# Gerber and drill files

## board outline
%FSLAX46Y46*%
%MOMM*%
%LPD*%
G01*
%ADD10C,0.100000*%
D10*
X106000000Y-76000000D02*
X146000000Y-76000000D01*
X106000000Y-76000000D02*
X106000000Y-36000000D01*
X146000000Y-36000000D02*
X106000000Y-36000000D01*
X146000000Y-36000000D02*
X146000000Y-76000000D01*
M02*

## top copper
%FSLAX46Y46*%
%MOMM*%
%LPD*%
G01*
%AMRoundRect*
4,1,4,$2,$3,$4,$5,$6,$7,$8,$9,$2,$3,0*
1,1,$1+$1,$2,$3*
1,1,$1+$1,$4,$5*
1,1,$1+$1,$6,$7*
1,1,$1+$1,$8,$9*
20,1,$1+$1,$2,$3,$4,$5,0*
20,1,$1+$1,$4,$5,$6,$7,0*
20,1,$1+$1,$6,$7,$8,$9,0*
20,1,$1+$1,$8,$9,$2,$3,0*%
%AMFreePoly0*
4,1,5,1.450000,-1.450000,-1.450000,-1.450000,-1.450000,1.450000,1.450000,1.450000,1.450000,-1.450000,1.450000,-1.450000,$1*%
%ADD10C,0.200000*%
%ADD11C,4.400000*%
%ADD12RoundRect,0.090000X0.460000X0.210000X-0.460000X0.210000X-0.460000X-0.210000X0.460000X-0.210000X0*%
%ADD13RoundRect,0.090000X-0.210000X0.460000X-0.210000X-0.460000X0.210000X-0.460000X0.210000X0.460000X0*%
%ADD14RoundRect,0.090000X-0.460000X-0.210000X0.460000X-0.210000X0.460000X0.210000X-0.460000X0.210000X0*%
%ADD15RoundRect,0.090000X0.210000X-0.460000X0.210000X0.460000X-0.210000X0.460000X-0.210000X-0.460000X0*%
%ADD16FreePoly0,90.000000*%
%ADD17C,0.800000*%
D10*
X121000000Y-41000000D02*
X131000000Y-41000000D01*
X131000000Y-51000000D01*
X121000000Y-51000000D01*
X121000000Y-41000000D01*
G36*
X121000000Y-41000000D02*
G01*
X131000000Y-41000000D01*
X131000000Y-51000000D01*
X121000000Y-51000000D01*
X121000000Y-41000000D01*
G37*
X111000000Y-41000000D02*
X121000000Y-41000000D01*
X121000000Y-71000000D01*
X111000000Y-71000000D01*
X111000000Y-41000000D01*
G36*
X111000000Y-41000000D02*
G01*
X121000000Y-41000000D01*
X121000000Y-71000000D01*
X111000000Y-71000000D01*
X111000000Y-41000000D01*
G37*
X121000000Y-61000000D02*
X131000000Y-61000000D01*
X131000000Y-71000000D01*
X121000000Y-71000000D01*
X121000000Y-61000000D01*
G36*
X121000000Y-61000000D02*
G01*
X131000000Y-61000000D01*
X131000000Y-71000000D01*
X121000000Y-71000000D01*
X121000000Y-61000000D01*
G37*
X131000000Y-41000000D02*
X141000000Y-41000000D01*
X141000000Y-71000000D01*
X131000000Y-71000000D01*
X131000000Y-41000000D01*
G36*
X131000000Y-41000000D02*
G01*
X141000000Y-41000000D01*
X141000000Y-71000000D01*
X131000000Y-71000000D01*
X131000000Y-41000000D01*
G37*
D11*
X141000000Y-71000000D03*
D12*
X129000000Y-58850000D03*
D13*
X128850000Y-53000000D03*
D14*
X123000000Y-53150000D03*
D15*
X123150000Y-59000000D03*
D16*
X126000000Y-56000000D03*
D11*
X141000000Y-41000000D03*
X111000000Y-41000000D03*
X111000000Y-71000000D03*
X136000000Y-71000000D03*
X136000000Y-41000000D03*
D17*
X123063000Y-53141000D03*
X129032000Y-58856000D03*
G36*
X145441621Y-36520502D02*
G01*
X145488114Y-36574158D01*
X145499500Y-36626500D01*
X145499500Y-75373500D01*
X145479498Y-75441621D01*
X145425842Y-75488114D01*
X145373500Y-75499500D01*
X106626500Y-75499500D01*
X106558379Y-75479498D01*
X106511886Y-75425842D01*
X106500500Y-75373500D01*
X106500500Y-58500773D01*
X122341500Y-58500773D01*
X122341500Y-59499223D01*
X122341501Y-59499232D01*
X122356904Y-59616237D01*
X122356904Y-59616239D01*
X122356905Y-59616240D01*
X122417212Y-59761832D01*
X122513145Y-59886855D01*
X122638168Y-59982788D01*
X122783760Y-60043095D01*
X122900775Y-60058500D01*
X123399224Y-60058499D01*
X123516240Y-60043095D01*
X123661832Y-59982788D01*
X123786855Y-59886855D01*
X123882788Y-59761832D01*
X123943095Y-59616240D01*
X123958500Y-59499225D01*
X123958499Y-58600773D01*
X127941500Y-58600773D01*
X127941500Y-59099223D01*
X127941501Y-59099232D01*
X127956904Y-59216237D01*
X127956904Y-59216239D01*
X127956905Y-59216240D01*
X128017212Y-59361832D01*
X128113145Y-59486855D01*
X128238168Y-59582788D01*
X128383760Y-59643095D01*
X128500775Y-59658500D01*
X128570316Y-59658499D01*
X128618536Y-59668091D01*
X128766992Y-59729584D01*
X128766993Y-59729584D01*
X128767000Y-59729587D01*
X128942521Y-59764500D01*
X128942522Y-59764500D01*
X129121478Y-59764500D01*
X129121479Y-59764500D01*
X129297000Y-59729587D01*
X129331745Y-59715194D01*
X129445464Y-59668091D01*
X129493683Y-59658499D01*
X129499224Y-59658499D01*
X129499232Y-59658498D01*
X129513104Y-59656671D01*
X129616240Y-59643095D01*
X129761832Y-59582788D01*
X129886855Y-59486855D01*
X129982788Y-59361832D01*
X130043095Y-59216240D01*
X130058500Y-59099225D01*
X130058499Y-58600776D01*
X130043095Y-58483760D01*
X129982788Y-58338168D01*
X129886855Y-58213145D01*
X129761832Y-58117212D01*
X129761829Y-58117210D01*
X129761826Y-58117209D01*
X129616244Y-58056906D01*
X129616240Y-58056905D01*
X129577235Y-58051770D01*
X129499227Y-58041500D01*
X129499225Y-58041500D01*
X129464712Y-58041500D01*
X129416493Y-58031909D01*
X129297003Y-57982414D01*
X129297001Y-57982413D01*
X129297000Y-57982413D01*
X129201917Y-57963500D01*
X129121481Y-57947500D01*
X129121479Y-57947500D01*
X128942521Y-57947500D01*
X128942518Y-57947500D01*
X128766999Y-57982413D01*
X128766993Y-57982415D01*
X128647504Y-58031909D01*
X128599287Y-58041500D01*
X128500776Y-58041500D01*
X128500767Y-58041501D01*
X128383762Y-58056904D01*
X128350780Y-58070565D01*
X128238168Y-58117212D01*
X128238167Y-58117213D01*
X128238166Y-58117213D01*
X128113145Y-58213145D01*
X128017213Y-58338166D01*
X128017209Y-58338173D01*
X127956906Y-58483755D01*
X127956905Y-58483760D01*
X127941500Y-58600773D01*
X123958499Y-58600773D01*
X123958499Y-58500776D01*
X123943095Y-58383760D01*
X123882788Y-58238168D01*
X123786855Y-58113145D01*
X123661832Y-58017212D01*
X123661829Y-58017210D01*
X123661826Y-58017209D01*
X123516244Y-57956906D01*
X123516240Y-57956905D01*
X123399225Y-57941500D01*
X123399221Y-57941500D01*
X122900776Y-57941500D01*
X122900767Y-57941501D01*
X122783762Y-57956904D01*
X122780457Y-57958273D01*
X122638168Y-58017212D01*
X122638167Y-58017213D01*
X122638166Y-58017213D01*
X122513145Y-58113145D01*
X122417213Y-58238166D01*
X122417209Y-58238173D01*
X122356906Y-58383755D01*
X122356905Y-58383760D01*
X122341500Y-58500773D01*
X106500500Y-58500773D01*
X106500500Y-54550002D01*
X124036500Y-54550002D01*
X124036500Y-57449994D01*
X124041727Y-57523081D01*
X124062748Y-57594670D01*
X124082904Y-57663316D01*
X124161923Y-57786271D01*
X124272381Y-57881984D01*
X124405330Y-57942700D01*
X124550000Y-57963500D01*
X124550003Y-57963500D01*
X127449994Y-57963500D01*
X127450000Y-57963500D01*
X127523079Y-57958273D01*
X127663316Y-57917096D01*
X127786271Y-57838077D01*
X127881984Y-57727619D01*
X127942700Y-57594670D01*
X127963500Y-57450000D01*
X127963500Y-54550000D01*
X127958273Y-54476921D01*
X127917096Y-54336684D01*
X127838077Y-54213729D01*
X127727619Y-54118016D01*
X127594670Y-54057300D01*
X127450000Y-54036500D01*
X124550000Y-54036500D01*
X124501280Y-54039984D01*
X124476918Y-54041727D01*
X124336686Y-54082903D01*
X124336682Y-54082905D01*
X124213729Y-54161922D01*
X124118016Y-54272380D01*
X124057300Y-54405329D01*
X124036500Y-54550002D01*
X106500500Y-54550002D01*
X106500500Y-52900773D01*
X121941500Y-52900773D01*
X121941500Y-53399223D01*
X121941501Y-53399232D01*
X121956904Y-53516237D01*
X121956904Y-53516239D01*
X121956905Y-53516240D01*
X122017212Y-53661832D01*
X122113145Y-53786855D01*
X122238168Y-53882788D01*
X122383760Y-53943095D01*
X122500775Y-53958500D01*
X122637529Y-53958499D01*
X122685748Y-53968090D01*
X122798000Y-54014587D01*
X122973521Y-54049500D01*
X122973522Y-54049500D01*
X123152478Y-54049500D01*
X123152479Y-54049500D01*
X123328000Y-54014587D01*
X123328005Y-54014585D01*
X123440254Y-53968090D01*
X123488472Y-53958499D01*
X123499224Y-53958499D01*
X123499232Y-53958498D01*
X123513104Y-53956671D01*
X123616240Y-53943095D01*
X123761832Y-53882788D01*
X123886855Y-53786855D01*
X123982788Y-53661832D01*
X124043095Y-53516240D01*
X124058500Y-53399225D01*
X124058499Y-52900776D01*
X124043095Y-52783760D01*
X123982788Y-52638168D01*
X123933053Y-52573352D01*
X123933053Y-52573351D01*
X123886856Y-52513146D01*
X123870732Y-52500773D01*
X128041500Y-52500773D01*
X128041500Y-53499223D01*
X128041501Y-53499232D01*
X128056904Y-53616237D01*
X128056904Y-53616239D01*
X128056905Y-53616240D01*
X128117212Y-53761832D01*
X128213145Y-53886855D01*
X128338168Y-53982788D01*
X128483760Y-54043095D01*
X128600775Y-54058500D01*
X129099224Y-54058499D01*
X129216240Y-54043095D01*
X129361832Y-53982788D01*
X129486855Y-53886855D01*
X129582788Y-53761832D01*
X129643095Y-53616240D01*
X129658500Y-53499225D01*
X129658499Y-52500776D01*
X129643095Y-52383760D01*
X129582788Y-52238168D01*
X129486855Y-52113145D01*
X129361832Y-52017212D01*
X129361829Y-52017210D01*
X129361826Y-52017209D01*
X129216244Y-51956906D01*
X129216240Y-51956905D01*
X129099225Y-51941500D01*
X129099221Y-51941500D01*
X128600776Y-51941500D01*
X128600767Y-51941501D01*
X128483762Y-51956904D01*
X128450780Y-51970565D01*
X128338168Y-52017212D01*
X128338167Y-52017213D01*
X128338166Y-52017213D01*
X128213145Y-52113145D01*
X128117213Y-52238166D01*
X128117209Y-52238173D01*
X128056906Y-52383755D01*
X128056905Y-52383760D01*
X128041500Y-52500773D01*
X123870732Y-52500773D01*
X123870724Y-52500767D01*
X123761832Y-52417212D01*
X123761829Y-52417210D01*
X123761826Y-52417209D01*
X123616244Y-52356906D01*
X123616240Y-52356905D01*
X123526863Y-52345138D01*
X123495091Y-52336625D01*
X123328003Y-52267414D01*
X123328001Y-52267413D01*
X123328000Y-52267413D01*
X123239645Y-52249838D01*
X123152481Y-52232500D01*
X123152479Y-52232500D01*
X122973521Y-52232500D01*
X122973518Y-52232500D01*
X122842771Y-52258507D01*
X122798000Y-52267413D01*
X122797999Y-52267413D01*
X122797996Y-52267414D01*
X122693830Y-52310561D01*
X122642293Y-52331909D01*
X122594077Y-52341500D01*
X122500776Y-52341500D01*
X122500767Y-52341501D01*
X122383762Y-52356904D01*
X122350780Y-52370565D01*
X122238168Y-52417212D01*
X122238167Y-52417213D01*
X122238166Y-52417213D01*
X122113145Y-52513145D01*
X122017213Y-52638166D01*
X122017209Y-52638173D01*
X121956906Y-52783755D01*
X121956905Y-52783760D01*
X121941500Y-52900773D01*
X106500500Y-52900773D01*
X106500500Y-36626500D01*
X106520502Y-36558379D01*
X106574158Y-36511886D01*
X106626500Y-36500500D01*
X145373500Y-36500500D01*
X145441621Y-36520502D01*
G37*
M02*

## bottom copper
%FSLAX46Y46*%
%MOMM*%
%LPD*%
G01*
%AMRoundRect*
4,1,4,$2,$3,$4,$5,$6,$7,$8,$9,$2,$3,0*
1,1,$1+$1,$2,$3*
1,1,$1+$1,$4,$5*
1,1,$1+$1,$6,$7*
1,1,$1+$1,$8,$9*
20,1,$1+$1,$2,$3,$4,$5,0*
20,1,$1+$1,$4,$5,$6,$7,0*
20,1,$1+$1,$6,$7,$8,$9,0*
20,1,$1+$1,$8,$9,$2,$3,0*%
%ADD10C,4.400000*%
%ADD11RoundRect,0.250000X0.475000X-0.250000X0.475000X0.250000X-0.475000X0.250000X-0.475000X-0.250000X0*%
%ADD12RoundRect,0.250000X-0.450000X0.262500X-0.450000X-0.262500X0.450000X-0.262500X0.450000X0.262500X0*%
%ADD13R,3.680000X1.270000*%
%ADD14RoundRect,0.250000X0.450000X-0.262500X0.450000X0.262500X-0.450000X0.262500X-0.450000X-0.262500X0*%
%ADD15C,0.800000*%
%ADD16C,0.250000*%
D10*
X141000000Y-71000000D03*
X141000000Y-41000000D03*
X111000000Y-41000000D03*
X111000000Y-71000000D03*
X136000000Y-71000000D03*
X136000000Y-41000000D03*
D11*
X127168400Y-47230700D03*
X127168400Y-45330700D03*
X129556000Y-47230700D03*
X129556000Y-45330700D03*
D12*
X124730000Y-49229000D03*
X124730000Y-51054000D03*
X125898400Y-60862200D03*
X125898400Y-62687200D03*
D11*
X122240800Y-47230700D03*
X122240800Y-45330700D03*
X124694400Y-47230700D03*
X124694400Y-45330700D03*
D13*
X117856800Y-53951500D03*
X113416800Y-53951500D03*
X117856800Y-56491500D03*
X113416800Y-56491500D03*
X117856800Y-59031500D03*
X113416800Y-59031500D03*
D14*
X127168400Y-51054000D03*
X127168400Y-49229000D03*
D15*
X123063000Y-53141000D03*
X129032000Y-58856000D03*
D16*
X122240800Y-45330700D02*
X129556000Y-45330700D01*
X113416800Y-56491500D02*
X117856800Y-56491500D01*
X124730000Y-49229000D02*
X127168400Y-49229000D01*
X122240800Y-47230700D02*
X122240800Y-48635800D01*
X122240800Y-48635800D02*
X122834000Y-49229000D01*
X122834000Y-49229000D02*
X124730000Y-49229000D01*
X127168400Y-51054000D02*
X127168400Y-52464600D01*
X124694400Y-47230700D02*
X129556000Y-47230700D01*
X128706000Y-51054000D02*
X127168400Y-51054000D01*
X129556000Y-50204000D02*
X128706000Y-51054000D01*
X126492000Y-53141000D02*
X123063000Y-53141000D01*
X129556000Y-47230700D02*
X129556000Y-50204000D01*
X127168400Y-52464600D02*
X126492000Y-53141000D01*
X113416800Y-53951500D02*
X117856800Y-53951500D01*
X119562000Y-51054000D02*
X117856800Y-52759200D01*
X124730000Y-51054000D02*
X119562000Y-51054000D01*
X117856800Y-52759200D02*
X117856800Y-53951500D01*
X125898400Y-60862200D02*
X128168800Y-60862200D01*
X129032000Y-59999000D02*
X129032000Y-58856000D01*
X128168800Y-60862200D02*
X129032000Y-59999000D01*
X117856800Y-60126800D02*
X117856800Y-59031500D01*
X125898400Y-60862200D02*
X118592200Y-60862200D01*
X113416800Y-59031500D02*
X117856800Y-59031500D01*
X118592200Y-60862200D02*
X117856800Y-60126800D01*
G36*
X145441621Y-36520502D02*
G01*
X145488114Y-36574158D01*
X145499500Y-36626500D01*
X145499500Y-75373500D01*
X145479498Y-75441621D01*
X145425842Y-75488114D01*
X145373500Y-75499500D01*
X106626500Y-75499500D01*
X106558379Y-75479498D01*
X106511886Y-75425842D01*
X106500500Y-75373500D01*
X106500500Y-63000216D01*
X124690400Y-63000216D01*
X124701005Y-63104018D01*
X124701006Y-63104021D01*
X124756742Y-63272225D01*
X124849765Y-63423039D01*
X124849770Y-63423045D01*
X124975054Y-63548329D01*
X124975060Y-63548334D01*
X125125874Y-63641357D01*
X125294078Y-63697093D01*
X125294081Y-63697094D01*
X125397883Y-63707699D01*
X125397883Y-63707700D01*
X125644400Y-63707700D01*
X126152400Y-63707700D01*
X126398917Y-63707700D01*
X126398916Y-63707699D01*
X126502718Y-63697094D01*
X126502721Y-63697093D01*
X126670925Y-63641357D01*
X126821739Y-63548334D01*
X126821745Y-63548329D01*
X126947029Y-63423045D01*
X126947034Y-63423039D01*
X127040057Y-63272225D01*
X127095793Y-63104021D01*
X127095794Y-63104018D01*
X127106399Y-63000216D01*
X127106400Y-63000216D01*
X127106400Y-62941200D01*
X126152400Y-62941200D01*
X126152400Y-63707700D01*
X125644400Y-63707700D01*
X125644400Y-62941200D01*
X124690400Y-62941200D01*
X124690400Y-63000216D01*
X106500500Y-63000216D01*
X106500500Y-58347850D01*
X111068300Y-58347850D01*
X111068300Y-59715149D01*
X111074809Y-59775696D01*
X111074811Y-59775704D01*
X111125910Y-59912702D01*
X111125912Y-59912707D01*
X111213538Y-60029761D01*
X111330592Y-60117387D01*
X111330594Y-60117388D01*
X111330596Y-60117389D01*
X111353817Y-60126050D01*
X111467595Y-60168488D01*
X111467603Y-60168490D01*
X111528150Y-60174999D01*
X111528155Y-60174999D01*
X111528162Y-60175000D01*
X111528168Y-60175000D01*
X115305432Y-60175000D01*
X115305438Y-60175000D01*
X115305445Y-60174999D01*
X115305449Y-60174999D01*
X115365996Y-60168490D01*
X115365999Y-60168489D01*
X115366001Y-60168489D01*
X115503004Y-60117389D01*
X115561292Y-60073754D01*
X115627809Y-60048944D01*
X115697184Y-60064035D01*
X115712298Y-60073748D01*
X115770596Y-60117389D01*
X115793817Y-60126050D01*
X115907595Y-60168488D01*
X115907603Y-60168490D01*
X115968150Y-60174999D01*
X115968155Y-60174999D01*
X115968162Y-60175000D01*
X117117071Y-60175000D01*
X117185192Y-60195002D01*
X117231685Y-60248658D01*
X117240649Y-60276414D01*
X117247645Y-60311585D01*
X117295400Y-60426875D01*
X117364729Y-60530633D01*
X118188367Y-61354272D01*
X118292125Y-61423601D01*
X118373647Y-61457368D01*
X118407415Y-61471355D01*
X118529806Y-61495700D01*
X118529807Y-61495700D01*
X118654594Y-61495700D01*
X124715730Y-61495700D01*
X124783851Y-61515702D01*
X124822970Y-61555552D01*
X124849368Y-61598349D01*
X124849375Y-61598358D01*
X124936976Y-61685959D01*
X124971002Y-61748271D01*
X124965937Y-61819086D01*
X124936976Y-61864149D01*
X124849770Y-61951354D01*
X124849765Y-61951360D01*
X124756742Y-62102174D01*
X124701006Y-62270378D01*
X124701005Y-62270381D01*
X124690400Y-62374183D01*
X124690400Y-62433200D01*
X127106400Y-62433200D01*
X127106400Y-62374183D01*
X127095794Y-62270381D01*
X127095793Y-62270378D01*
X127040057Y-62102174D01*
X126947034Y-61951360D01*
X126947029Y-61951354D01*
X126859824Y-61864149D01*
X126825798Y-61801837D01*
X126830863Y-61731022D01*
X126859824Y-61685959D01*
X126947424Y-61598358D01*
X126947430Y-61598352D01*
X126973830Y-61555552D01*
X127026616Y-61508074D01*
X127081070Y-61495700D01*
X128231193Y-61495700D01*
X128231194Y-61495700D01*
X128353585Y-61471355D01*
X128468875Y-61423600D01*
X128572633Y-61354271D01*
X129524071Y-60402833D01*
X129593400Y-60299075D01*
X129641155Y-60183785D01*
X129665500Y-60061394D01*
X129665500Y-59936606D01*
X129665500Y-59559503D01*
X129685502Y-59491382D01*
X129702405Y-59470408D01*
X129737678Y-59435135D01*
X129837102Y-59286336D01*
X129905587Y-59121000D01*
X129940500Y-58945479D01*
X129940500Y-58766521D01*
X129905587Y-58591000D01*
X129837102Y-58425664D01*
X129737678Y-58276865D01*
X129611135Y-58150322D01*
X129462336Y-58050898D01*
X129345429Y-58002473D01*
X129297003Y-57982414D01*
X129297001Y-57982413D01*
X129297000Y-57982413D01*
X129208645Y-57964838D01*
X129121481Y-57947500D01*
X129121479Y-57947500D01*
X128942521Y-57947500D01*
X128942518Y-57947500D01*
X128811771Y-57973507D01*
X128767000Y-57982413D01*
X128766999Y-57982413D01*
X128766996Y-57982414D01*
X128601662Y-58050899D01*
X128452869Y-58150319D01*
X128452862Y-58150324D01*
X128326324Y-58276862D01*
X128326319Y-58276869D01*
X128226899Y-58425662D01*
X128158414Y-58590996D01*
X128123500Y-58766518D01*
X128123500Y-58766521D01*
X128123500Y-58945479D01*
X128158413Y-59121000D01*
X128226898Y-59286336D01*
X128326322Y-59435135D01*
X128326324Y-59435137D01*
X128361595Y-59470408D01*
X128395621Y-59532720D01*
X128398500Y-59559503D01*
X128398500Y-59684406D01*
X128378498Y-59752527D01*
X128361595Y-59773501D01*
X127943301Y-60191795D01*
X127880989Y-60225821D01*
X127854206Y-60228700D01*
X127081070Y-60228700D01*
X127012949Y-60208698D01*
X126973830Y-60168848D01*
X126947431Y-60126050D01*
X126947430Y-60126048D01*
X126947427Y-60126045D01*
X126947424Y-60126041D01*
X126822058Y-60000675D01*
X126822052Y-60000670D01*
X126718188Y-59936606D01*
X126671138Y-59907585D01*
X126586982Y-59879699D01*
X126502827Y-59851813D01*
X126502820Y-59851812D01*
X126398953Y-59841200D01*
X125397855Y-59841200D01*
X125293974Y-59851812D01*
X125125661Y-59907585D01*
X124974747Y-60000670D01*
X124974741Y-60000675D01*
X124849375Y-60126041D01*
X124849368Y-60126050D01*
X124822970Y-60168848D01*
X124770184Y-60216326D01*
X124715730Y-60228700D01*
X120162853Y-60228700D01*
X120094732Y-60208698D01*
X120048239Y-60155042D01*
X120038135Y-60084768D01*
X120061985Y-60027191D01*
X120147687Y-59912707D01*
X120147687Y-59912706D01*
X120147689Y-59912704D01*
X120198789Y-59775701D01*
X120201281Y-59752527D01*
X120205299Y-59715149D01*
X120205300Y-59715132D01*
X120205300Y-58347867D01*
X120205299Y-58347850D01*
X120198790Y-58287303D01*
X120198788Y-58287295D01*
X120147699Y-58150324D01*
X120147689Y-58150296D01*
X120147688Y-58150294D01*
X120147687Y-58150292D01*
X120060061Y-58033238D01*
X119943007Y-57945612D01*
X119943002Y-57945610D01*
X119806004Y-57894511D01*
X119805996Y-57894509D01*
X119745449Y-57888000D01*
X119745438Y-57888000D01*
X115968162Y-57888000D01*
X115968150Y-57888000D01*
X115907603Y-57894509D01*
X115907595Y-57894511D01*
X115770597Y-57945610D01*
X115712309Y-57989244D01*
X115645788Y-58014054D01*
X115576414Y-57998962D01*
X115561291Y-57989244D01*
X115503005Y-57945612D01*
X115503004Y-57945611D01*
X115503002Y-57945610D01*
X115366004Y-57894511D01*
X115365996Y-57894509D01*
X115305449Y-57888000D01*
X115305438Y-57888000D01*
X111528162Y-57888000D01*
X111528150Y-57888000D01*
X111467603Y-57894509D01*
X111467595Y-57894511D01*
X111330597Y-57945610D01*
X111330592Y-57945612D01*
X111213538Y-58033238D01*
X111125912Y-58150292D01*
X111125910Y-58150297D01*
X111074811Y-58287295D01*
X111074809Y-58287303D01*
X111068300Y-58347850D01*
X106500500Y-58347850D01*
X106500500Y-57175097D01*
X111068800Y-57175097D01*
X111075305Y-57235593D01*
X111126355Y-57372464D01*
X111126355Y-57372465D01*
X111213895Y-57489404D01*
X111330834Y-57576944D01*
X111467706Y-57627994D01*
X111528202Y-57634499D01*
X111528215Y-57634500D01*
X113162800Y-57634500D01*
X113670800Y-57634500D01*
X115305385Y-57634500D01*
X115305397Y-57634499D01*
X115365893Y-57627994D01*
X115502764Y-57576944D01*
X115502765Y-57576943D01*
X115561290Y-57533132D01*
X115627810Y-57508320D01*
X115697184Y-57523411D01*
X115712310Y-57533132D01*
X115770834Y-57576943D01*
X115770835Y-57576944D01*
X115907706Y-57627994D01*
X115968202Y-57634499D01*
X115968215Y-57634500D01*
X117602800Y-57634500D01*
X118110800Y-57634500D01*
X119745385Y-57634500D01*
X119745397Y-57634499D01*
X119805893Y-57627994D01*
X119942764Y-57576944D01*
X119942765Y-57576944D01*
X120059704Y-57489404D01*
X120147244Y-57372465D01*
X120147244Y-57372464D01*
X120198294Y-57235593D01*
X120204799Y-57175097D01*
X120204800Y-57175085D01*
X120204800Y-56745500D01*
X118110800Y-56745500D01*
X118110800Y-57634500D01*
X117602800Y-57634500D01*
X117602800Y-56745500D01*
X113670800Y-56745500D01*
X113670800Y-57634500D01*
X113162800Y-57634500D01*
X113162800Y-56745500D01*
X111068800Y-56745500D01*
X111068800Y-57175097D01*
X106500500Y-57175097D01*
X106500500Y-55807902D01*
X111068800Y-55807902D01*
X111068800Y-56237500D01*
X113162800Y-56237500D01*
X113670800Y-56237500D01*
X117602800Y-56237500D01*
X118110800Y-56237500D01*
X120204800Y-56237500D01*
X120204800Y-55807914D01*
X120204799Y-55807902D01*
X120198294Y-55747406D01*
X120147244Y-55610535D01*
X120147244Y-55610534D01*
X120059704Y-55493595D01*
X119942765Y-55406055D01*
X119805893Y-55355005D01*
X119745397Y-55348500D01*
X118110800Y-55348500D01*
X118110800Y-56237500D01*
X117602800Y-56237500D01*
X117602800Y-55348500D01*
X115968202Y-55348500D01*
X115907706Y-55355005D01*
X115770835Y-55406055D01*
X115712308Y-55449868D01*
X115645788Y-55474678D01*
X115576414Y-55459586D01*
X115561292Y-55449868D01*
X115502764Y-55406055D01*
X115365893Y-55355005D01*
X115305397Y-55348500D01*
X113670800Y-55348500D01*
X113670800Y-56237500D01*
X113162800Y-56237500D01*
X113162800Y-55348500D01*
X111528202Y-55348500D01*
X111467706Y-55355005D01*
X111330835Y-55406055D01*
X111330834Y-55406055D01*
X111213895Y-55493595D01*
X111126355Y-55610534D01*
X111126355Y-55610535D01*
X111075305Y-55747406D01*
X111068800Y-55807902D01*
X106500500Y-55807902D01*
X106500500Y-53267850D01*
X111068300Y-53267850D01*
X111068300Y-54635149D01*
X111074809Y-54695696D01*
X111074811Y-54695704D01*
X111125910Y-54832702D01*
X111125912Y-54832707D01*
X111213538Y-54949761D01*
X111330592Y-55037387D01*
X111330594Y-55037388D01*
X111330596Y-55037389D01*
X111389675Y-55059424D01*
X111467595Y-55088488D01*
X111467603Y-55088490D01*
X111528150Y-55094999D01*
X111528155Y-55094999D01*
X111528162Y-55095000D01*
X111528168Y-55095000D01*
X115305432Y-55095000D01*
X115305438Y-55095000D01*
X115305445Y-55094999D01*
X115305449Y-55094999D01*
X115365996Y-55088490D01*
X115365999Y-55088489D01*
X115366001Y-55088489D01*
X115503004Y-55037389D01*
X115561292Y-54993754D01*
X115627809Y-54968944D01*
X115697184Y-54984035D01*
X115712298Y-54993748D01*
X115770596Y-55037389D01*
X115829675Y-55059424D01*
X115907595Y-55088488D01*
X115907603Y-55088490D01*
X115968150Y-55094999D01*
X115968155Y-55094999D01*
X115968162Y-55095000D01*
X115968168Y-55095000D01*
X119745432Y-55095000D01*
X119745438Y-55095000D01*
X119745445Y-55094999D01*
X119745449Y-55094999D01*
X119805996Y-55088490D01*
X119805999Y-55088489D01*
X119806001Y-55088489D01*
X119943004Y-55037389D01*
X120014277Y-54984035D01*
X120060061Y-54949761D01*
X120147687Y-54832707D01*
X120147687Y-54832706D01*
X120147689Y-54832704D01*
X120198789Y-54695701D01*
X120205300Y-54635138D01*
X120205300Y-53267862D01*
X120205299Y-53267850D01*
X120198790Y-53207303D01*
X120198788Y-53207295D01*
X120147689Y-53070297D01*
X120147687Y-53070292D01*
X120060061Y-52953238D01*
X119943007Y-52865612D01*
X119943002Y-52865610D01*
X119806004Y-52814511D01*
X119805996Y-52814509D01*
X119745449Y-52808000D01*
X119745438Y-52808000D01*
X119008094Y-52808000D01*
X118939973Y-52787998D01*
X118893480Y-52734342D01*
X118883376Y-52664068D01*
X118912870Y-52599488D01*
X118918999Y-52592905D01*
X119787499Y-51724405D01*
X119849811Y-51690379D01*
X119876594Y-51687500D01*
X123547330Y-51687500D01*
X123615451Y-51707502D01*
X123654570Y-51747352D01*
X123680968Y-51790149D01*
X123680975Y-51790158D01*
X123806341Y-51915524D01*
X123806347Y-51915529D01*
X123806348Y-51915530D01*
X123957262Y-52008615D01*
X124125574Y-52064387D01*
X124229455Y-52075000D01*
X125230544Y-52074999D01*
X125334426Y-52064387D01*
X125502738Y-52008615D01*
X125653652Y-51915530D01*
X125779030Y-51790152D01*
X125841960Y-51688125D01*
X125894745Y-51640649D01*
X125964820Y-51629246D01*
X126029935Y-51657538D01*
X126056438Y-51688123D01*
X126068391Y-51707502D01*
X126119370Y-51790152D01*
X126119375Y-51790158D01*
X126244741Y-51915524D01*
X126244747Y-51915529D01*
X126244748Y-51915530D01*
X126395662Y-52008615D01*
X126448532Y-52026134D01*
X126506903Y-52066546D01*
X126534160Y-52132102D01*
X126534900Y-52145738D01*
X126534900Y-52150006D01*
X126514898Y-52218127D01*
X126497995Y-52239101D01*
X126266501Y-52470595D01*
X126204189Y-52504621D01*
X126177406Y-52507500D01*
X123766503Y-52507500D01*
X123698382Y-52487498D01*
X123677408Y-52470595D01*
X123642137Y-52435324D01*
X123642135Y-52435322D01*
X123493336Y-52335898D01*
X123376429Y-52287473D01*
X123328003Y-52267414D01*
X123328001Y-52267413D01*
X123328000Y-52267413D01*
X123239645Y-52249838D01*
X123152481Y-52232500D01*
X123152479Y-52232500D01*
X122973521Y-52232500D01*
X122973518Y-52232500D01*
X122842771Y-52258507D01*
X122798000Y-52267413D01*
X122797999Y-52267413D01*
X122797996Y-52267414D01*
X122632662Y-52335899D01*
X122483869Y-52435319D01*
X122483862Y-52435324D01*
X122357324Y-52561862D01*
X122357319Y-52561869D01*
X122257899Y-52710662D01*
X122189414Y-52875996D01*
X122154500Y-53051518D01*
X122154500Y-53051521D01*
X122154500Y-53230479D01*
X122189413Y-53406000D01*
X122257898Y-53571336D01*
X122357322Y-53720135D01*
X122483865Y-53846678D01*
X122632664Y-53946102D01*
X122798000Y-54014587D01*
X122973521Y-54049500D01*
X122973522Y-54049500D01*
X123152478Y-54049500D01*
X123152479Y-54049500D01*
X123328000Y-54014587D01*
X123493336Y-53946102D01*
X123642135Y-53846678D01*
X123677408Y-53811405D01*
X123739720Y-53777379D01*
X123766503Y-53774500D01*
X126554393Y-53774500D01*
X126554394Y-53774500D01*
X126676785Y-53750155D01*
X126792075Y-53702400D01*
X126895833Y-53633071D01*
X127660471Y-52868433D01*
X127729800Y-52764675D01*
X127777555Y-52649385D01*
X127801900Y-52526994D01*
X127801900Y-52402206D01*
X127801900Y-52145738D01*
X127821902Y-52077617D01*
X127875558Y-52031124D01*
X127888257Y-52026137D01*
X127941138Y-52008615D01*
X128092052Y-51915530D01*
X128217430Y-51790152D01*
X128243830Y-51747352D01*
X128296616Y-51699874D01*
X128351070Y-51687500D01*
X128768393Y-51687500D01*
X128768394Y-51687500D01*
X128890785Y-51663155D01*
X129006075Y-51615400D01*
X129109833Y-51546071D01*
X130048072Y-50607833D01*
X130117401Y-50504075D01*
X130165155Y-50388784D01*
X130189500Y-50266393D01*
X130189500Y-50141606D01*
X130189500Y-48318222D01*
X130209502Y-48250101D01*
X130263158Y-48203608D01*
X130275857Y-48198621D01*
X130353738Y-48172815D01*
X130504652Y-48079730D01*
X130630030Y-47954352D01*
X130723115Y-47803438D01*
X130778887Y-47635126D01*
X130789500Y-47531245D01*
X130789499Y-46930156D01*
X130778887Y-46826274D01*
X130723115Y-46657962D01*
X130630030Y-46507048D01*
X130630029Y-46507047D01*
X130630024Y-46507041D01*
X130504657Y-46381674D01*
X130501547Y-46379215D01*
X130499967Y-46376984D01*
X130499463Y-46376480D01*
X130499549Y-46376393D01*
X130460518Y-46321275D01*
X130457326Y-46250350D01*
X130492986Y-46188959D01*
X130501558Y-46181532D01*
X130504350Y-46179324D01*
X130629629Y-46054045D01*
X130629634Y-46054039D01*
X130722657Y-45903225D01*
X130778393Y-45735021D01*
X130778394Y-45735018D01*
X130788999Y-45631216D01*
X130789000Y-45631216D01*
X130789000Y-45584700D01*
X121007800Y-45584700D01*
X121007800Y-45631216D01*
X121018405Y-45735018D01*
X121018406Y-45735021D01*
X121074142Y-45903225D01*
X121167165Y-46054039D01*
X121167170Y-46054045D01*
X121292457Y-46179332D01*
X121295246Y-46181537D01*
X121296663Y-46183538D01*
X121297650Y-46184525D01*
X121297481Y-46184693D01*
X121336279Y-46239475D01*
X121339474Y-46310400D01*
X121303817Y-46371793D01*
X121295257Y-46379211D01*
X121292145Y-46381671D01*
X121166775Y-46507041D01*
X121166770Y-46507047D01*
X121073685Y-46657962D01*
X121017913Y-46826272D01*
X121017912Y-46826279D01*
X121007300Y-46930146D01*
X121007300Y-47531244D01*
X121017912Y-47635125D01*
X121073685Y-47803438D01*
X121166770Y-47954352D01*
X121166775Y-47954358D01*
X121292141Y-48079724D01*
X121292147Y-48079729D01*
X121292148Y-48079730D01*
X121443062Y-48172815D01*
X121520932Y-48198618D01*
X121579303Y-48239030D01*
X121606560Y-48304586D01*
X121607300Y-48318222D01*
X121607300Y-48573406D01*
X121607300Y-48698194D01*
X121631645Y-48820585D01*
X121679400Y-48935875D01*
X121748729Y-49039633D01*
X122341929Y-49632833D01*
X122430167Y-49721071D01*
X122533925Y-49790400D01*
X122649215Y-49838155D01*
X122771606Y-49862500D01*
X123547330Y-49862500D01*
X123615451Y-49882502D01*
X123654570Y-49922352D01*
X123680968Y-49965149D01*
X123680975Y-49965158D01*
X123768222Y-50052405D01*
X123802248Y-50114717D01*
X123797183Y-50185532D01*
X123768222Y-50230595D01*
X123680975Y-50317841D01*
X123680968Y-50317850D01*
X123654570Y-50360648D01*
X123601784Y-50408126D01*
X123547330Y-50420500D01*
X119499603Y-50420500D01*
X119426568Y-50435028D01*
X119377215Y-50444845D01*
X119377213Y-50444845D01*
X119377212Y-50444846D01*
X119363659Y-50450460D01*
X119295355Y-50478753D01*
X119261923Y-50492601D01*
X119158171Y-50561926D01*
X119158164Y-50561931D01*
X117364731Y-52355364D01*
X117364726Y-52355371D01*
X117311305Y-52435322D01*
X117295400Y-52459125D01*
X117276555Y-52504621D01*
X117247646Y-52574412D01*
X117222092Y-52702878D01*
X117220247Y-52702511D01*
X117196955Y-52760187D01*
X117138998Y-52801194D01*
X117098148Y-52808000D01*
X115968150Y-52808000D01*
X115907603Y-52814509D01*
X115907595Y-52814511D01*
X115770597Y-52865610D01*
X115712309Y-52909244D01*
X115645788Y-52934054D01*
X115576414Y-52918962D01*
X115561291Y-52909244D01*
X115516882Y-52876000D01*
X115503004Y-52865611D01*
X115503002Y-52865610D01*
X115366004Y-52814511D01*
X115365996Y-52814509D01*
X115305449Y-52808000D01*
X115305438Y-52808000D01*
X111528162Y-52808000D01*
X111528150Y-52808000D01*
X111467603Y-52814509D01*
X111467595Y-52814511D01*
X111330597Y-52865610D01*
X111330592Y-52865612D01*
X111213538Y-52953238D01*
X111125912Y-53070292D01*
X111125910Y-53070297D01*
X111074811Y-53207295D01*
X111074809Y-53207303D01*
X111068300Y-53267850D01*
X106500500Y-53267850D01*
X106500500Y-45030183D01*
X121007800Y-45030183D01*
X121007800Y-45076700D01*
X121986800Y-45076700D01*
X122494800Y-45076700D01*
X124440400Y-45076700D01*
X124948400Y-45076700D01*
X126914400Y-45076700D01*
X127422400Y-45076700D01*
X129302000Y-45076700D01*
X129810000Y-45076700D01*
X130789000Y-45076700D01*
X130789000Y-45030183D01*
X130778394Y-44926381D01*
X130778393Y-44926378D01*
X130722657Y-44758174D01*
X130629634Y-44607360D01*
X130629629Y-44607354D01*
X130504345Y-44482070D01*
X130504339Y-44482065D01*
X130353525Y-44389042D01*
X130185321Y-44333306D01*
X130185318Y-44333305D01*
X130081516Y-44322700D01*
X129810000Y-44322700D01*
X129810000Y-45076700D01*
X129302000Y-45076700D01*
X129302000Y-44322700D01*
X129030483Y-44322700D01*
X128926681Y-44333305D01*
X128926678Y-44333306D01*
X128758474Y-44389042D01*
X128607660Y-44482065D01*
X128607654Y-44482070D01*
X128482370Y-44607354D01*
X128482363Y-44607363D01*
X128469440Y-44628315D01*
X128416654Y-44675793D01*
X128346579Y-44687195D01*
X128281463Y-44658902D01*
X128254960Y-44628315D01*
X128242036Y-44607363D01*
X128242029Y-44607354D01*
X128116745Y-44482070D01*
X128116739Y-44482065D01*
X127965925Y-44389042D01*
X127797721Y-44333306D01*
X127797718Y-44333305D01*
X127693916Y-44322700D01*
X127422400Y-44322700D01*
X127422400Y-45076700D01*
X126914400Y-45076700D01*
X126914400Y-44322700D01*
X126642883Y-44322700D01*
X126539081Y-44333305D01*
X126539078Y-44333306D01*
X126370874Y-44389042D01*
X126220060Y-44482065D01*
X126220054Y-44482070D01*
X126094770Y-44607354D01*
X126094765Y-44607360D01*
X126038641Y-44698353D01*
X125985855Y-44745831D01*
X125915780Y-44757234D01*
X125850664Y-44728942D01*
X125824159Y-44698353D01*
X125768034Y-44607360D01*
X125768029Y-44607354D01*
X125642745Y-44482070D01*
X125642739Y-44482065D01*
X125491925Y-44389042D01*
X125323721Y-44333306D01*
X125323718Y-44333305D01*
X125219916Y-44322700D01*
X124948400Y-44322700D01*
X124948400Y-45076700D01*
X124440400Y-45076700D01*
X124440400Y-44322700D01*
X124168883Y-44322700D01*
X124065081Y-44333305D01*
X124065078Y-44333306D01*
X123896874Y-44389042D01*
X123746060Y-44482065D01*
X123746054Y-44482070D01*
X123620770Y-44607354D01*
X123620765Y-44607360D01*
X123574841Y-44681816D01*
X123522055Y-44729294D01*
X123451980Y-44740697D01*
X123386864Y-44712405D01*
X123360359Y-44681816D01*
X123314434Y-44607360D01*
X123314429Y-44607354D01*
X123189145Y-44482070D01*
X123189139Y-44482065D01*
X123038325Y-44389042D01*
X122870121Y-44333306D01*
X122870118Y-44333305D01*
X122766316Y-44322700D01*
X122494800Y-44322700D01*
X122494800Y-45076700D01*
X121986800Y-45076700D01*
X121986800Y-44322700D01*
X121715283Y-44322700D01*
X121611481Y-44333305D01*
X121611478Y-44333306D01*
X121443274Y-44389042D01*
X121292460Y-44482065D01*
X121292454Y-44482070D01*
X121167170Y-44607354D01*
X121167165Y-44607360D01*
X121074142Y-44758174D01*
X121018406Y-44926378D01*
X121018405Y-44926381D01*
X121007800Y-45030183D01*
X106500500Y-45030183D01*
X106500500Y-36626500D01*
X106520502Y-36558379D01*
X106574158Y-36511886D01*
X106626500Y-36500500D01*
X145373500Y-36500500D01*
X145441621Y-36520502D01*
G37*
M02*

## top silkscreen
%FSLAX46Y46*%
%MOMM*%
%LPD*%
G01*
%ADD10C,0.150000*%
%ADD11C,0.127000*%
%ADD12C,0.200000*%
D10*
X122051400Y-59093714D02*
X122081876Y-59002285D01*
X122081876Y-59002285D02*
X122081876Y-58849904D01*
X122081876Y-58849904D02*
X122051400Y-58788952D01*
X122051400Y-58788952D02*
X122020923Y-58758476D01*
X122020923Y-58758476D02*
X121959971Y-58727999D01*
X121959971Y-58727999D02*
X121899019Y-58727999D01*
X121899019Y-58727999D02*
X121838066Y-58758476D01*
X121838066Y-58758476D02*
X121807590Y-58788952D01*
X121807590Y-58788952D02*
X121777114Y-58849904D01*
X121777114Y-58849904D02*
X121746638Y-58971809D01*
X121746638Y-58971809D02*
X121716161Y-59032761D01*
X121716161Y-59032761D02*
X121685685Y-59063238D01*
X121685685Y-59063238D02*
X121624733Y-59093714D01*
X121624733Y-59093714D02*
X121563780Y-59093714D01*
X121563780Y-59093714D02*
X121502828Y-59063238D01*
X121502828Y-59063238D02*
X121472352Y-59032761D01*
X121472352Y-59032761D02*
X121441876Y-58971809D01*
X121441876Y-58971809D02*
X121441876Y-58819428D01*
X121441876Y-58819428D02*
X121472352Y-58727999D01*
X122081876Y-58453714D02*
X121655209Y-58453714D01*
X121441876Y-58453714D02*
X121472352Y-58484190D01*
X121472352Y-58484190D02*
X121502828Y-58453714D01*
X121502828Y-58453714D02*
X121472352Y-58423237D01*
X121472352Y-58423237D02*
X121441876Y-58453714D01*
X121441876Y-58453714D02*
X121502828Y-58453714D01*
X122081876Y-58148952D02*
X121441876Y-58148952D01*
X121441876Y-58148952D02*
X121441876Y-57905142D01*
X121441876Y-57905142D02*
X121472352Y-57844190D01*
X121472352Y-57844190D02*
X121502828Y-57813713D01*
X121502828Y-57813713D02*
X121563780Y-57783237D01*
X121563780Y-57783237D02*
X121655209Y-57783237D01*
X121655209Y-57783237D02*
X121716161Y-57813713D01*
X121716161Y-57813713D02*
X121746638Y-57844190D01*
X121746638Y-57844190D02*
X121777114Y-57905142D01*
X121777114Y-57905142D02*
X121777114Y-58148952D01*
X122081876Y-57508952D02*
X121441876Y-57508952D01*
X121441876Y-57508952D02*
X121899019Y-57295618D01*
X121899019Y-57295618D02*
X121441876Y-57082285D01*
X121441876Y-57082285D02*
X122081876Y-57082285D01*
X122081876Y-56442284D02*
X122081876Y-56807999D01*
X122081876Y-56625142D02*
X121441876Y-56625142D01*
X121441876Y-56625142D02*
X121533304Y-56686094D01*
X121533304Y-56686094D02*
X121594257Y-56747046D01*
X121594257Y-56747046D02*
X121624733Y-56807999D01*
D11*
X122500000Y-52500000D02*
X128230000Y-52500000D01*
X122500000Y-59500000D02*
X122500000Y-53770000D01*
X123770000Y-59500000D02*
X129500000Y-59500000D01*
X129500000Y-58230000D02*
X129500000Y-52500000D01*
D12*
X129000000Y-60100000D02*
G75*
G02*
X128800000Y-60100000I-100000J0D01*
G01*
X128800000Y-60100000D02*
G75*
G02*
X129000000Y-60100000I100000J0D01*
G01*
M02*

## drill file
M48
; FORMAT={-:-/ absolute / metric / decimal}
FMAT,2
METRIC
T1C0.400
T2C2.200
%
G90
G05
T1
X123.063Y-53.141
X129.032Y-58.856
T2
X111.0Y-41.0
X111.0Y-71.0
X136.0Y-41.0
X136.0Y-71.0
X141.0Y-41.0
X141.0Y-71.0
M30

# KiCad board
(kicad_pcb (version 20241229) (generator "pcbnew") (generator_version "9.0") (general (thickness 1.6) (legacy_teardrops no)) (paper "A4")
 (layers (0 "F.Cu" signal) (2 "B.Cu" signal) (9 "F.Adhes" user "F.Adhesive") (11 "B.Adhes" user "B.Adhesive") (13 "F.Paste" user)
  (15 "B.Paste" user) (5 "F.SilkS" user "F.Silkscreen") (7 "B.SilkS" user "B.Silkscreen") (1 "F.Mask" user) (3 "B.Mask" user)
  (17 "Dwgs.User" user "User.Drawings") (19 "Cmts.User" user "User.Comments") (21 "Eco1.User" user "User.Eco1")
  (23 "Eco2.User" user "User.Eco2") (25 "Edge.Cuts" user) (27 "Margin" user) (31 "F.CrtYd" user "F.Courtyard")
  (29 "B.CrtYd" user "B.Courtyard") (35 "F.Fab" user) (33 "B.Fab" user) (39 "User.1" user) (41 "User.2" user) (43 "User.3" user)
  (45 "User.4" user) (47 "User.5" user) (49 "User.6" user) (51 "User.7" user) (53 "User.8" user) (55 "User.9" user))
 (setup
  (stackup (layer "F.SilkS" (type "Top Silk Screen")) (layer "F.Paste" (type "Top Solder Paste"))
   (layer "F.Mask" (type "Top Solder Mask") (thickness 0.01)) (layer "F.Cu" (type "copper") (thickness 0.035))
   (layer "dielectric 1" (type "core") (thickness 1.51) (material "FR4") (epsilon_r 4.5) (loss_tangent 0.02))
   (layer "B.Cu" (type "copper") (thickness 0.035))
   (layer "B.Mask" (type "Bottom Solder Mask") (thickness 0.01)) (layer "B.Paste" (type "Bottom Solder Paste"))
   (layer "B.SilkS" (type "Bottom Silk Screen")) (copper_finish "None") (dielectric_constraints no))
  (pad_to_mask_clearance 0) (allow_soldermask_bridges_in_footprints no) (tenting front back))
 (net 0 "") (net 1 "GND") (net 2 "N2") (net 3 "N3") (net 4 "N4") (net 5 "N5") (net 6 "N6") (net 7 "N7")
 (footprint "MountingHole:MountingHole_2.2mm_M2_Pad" (layer "F.Cu") (at 141 71)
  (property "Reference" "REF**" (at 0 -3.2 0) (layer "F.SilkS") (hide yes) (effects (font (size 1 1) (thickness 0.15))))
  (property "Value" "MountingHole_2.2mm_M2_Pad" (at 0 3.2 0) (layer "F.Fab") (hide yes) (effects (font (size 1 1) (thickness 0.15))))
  (pad "1" thru_hole circle (at 0 0) (size 4.4 4.4) (drill 2.2) (layers "*.Cu" "*.Mask") (remove_unused_layers no) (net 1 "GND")
   (zone_connect 2)))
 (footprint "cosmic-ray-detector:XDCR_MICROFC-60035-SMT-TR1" (layer "F.Cu") (at 126 56 90)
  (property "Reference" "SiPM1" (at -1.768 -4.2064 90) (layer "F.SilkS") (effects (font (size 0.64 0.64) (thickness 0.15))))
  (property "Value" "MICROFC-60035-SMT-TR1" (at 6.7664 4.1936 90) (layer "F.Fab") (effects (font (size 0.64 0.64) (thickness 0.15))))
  (fp_line (start 3.5 -3.5) (end 3.5 2.23) (stroke (width 0.127) (type solid)) (layer "F.SilkS"))
  (fp_line (start -3.5 -3.5) (end 2.23 -3.5) (stroke (width 0.127) (type solid)) (layer "F.SilkS"))
  (fp_line (start -3.5 -2.23) (end -3.5 3.5) (stroke (width 0.127) (type solid)) (layer "F.SilkS"))
  (fp_line (start -2.23 3.5) (end 3.5 3.5) (stroke (width 0.127) (type solid)) (layer "F.SilkS"))
  (fp_circle (center -4.1 2.9) (end -4 2.9) (stroke (width 0.2) (type solid)) (fill no) (layer "F.SilkS"))
  (pad "1" smd roundrect (at -2.85 3 180) (size 1.1 0.6) (layers "F.Cu" "F.Mask" "F.Paste") (roundrect_rratio 0.15) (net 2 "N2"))
  (pad "2" smd roundrect (at 3 2.85 270) (size 1.1 0.6) (layers "F.Cu" "F.Mask" "F.Paste") (roundrect_rratio 0.15) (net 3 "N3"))
  (pad "3" smd roundrect (at 2.85 -3) (size 1.1 0.6) (layers "F.Cu" "F.Mask" "F.Paste") (roundrect_rratio 0.15) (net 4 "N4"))
  (pad "4" smd roundrect (at -3 -2.85 90) (size 1.1 0.6) (layers "F.Cu" "F.Mask" "F.Paste") (roundrect_rratio 0.15))
  (pad "5" smd custom (at 0 0 90) (size 2.9 2.9) (layers "F.Cu") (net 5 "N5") (zone_connect 0) (options (clearance outline) (anchor rect))
   (primitives)))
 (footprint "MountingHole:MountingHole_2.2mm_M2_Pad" (layer "F.Cu") (at 141 41)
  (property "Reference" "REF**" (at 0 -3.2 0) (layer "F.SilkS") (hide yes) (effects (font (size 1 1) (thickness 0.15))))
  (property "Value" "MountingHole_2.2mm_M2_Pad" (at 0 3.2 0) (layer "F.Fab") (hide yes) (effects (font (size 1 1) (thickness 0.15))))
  (pad "1" thru_hole circle (at 0 0) (size 4.4 4.4) (drill 2.2) (layers "*.Cu" "*.Mask") (remove_unused_layers no) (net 1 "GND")
   (zone_connect 2)))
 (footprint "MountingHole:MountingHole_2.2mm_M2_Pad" (layer "F.Cu") (at 111 41)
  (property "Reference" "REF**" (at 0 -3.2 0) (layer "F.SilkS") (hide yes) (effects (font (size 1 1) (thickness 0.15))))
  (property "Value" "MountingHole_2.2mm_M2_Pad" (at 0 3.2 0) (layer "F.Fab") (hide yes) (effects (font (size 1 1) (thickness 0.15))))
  (pad "1" thru_hole circle (at 0 0) (size 4.4 4.4) (drill 2.2) (layers "*.Cu" "*.Mask") (remove_unused_layers no) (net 1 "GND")
   (zone_connect 2)))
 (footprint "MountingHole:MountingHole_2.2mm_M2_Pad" (layer "F.Cu") (at 111 71)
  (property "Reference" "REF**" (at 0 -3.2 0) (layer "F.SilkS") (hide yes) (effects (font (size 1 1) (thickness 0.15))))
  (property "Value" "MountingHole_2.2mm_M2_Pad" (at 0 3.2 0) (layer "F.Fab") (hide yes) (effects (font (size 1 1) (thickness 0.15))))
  (pad "1" thru_hole circle (at 0 0) (size 4.4 4.4) (drill 2.2) (layers "*.Cu" "*.Mask") (remove_unused_layers no) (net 1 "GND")
   (zone_connect 2)))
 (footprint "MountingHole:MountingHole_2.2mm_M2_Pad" (layer "F.Cu") (at 136 71)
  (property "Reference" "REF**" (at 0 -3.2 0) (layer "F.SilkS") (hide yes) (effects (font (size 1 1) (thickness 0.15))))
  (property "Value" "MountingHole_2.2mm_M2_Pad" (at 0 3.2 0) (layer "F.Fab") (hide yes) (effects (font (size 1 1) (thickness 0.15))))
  (pad "1" thru_hole circle (at 0 0) (size 4.4 4.4) (drill 2.2) (layers "*.Cu" "*.Mask") (remove_unused_layers no) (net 1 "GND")
   (zone_connect 2)))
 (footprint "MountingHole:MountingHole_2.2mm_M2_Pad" (layer "F.Cu") (at 136 41)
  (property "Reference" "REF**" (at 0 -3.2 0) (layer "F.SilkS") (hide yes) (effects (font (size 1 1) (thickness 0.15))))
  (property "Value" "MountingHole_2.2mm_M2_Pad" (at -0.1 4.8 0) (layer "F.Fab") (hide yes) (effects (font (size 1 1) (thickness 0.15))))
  (pad "1" thru_hole circle (at 0 0) (size 4.4 4.4) (drill 2.2) (layers "*.Cu" "*.Mask") (remove_unused_layers no) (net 1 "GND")
   (zone_connect 2)))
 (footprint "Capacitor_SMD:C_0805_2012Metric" (layer "B.Cu") (at 127.1684 46.2807 90)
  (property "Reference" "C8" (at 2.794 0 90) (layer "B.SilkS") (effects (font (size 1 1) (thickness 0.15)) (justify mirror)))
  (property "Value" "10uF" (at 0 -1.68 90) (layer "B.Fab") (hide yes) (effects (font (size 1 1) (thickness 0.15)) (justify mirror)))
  (pad "1" smd roundrect (at -0.95 0 90) (size 1 1.45) (layers "B.Cu" "B.Mask" "B.Paste") (roundrect_rratio 0.25) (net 4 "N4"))
  (pad "2" smd roundrect (at 0.95 0 90) (size 1 1.45) (layers "B.Cu" "B.Mask" "B.Paste") (roundrect_rratio 0.25) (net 1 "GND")))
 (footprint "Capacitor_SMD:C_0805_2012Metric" (layer "B.Cu") (at 129.556 46.2807 90)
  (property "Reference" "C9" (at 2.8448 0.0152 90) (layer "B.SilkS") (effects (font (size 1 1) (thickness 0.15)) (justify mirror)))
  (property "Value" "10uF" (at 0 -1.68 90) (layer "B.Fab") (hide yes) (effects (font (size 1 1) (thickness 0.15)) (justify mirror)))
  (pad "1" smd roundrect (at -0.95 0 90) (size 1 1.45) (layers "B.Cu" "B.Mask" "B.Paste") (roundrect_rratio 0.25) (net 4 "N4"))
  (pad "2" smd roundrect (at 0.95 0 90) (size 1 1.45) (layers "B.Cu" "B.Mask" "B.Paste") (roundrect_rratio 0.25) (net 1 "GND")))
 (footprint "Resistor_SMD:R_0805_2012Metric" (layer "B.Cu") (at 124.73 50.1415 -90)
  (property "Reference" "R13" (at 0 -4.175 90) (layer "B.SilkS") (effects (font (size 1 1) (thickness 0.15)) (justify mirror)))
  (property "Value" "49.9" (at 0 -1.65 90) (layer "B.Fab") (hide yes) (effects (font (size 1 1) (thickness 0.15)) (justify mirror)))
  (pad "1" smd roundrect (at -0.9125 0 270) (size 1.025 1.4) (layers "B.Cu" "B.Mask" "B.Paste") (roundrect_rratio 0.243902) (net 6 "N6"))
  (pad "2" smd roundrect (at 0.9125 0 270) (size 1.025 1.4) (layers "B.Cu" "B.Mask" "B.Paste") (roundrect_rratio 0.243902) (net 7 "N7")))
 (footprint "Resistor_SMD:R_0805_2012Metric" (layer "B.Cu") (at 125.8984 61.7747 -90)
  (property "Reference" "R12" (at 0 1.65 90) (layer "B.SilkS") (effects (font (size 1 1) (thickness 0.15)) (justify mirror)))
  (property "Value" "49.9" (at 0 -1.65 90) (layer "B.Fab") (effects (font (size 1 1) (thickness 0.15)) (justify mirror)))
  (pad "1" smd roundrect (at -0.9125 0 270) (size 1.025 1.4) (layers "B.Cu" "B.Mask" "B.Paste") (roundrect_rratio 0.243902) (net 2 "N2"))
  (pad "2" smd roundrect (at 0.9125 0 270) (size 1.025 1.4) (layers "B.Cu" "B.Mask" "B.Paste") (roundrect_rratio 0.243902) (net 1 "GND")))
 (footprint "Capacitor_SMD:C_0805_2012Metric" (layer "B.Cu") (at 122.2408 46.2807 90)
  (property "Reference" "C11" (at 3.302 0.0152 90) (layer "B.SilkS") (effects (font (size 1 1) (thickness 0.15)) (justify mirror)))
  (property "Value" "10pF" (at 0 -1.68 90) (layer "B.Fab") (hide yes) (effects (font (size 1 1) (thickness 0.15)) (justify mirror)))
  (pad "1" smd roundrect (at -0.95 0 90) (size 1 1.45) (layers "B.Cu" "B.Mask" "B.Paste") (roundrect_rratio 0.25) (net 6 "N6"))
  (pad "2" smd roundrect (at 0.95 0 90) (size 1 1.45) (layers "B.Cu" "B.Mask" "B.Paste") (roundrect_rratio 0.25) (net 1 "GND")))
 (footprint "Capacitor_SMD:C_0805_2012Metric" (layer "B.Cu") (at 124.6944 46.2807 90)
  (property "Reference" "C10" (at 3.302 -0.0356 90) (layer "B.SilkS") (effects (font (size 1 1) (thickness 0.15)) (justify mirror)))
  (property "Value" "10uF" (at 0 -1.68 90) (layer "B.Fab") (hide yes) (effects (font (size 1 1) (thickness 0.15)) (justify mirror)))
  (pad "1" smd roundrect (at -0.95 0 90) (size 1 1.45) (layers "B.Cu" "B.Mask" "B.Paste") (roundrect_rratio 0.25) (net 4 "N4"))
  (pad "2" smd roundrect (at 0.95 0 90) (size 1 1.45) (layers "B.Cu" "B.Mask" "B.Paste") (roundrect_rratio 0.25) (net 1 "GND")))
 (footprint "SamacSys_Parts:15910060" (layer "B.Cu") (at 115.6368 56.4915 -90)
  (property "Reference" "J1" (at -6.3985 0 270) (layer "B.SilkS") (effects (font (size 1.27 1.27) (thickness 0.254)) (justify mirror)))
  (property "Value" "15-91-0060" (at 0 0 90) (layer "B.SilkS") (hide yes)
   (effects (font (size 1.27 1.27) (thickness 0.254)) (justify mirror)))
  (pad "1" smd rect (at -2.54 -2.22 270) (size 1.27 3.68) (layers "B.Cu" "B.Mask" "B.Paste") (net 7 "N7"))
  (pad "2" smd rect (at -2.54 2.22 270) (size 1.27 3.68) (layers "B.Cu" "B.Mask" "B.Paste") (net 7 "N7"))
  (pad "3" smd rect (at 0 -2.22 270) (size 1.27 3.68) (layers "B.Cu" "B.Mask" "B.Paste") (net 1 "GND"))
  (pad "4" smd rect (at 0 2.22 270) (size 1.27 3.68) (layers "B.Cu" "B.Mask" "B.Paste") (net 1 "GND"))
  (pad "5" smd rect (at 2.54 -2.22 270) (size 1.27 3.68) (layers "B.Cu" "B.Mask" "B.Paste") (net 2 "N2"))
  (pad "6" smd rect (at 2.54 2.22 270) (size 1.27 3.68) (layers "B.Cu" "B.Mask" "B.Paste") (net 2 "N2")))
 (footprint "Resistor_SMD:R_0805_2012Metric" (layer "B.Cu") (at 127.1684 50.1415 90)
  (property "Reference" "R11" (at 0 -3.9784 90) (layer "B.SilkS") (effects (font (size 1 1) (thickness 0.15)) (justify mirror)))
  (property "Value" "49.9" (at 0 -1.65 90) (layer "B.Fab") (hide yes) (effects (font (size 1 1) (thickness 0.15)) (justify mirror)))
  (pad "1" smd roundrect (at -0.9125 0 90) (size 1.025 1.4) (layers "B.Cu" "B.Mask" "B.Paste") (roundrect_rratio 0.243902) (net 4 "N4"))
  (pad "2" smd roundrect (at 0.9125 0 90) (size 1.025 1.4) (layers "B.Cu" "B.Mask" "B.Paste") (roundrect_rratio 0.243902) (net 6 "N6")))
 (gr_rect (start 121 41) (end 131 51) (stroke (width 0.2) (type solid)) (fill yes) (layer "F.Cu") (net 1))
 (gr_rect (start 111 41) (end 121 71) (stroke (width 0.2) (type solid)) (fill yes) (layer "F.Cu") (net 1))
 (gr_rect (start 121 61) (end 131 71) (stroke (width 0.2) (type solid)) (fill yes) (layer "F.Cu") (net 1))
 (gr_rect (start 131 41) (end 141 71) (stroke (width 0.2) (type solid)) (fill yes) (layer "F.Cu") (net 1))
 (gr_line (start 106 76) (end 146 76) (stroke (width 0.1) (type solid)) (layer "Edge.Cuts"))
 (gr_line (start 106 76) (end 106 36) (stroke (width 0.1) (type solid)) (layer "Edge.Cuts"))
 (gr_line (start 146 36) (end 106 36) (stroke (width 0.1) (type solid)) (layer "Edge.Cuts"))
 (gr_line (start 146 36) (end 146 76) (stroke (width 0.1) (type solid)) (layer "Edge.Cuts"))
 (segment (start 122.2408 45.3307) (end 129.556 45.3307) (width 0.25) (layer "B.Cu") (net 1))
 (segment (start 113.4168 56.4915) (end 117.8568 56.4915) (width 0.25) (layer "B.Cu") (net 1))
 (segment (start 124.73 49.229) (end 127.1684 49.229) (width 0.25) (layer "B.Cu") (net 6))
 (segment (start 122.2408 47.2307) (end 122.2408 48.6358) (width 0.25) (layer "B.Cu") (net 6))
 (segment (start 122.2408 48.6358) (end 122.834 49.229) (width 0.25) (layer "B.Cu") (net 6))
 (segment (start 122.834 49.229) (end 124.73 49.229) (width 0.25) (layer "B.Cu") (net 6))
 (via (at 123.063 53.141) (size 0.8) (drill 0.4) (layers "F.Cu" "B.Cu") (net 4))
 (segment (start 127.1684 51.054) (end 127.1684 52.4646) (width 0.25) (layer "B.Cu") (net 4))
 (segment (start 124.6944 47.2307) (end 129.556 47.2307) (width 0.25) (layer "B.Cu") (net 4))
 (segment (start 128.706 51.054) (end 127.1684 51.054) (width 0.25) (layer "B.Cu") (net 4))
 (segment (start 129.556 50.204) (end 128.706 51.054) (width 0.25) (layer "B.Cu") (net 4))
 (segment (start 126.492 53.141) (end 123.063 53.141) (width 0.25) (layer "B.Cu") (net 4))
 (segment (start 129.556 47.2307) (end 129.556 50.204) (width 0.25) (layer "B.Cu") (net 4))
 (segment (start 127.1684 52.4646) (end 126.492 53.141) (width 0.25) (layer "B.Cu") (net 4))
 (segment (start 113.4168 53.9515) (end 117.8568 53.9515) (width 0.25) (layer "B.Cu") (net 7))
 (segment (start 119.562 51.054) (end 117.8568 52.7592) (width 0.25) (layer "B.Cu") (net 7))
 (segment (start 124.73 51.054) (end 119.562 51.054) (width 0.25) (layer "B.Cu") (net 7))
 (segment (start 117.8568 52.7592) (end 117.8568 53.9515) (width 0.25) (layer "B.Cu") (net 7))
 (via (at 129.032 58.856) (size 0.8) (drill 0.4) (layers "F.Cu" "B.Cu") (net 2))
 (segment (start 125.8984 60.8622) (end 128.1688 60.8622) (width 0.25) (layer "B.Cu") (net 2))
 (segment (start 129.032 59.999) (end 129.032 58.856) (width 0.25) (layer "B.Cu") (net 2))
 (segment (start 128.1688 60.8622) (end 129.032 59.999) (width 0.25) (layer "B.Cu") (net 2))
 (segment (start 117.8568 60.1268) (end 117.8568 59.0315) (width 0.25) (layer "B.Cu") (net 2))
 (segment (start 125.8984 60.8622) (end 118.5922 60.8622) (width 0.25) (layer "B.Cu") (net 2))
 (segment (start 113.4168 59.0315) (end 117.8568 59.0315) (width 0.25) (layer "B.Cu") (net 2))
 (segment (start 118.5922 60.8622) (end 117.8568 60.1268) (width 0.25) (layer "B.Cu") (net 2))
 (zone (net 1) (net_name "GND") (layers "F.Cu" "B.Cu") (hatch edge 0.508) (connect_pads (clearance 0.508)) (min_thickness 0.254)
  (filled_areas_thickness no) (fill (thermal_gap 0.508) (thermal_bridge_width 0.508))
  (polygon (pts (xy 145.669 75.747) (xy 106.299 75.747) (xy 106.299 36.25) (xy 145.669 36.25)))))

